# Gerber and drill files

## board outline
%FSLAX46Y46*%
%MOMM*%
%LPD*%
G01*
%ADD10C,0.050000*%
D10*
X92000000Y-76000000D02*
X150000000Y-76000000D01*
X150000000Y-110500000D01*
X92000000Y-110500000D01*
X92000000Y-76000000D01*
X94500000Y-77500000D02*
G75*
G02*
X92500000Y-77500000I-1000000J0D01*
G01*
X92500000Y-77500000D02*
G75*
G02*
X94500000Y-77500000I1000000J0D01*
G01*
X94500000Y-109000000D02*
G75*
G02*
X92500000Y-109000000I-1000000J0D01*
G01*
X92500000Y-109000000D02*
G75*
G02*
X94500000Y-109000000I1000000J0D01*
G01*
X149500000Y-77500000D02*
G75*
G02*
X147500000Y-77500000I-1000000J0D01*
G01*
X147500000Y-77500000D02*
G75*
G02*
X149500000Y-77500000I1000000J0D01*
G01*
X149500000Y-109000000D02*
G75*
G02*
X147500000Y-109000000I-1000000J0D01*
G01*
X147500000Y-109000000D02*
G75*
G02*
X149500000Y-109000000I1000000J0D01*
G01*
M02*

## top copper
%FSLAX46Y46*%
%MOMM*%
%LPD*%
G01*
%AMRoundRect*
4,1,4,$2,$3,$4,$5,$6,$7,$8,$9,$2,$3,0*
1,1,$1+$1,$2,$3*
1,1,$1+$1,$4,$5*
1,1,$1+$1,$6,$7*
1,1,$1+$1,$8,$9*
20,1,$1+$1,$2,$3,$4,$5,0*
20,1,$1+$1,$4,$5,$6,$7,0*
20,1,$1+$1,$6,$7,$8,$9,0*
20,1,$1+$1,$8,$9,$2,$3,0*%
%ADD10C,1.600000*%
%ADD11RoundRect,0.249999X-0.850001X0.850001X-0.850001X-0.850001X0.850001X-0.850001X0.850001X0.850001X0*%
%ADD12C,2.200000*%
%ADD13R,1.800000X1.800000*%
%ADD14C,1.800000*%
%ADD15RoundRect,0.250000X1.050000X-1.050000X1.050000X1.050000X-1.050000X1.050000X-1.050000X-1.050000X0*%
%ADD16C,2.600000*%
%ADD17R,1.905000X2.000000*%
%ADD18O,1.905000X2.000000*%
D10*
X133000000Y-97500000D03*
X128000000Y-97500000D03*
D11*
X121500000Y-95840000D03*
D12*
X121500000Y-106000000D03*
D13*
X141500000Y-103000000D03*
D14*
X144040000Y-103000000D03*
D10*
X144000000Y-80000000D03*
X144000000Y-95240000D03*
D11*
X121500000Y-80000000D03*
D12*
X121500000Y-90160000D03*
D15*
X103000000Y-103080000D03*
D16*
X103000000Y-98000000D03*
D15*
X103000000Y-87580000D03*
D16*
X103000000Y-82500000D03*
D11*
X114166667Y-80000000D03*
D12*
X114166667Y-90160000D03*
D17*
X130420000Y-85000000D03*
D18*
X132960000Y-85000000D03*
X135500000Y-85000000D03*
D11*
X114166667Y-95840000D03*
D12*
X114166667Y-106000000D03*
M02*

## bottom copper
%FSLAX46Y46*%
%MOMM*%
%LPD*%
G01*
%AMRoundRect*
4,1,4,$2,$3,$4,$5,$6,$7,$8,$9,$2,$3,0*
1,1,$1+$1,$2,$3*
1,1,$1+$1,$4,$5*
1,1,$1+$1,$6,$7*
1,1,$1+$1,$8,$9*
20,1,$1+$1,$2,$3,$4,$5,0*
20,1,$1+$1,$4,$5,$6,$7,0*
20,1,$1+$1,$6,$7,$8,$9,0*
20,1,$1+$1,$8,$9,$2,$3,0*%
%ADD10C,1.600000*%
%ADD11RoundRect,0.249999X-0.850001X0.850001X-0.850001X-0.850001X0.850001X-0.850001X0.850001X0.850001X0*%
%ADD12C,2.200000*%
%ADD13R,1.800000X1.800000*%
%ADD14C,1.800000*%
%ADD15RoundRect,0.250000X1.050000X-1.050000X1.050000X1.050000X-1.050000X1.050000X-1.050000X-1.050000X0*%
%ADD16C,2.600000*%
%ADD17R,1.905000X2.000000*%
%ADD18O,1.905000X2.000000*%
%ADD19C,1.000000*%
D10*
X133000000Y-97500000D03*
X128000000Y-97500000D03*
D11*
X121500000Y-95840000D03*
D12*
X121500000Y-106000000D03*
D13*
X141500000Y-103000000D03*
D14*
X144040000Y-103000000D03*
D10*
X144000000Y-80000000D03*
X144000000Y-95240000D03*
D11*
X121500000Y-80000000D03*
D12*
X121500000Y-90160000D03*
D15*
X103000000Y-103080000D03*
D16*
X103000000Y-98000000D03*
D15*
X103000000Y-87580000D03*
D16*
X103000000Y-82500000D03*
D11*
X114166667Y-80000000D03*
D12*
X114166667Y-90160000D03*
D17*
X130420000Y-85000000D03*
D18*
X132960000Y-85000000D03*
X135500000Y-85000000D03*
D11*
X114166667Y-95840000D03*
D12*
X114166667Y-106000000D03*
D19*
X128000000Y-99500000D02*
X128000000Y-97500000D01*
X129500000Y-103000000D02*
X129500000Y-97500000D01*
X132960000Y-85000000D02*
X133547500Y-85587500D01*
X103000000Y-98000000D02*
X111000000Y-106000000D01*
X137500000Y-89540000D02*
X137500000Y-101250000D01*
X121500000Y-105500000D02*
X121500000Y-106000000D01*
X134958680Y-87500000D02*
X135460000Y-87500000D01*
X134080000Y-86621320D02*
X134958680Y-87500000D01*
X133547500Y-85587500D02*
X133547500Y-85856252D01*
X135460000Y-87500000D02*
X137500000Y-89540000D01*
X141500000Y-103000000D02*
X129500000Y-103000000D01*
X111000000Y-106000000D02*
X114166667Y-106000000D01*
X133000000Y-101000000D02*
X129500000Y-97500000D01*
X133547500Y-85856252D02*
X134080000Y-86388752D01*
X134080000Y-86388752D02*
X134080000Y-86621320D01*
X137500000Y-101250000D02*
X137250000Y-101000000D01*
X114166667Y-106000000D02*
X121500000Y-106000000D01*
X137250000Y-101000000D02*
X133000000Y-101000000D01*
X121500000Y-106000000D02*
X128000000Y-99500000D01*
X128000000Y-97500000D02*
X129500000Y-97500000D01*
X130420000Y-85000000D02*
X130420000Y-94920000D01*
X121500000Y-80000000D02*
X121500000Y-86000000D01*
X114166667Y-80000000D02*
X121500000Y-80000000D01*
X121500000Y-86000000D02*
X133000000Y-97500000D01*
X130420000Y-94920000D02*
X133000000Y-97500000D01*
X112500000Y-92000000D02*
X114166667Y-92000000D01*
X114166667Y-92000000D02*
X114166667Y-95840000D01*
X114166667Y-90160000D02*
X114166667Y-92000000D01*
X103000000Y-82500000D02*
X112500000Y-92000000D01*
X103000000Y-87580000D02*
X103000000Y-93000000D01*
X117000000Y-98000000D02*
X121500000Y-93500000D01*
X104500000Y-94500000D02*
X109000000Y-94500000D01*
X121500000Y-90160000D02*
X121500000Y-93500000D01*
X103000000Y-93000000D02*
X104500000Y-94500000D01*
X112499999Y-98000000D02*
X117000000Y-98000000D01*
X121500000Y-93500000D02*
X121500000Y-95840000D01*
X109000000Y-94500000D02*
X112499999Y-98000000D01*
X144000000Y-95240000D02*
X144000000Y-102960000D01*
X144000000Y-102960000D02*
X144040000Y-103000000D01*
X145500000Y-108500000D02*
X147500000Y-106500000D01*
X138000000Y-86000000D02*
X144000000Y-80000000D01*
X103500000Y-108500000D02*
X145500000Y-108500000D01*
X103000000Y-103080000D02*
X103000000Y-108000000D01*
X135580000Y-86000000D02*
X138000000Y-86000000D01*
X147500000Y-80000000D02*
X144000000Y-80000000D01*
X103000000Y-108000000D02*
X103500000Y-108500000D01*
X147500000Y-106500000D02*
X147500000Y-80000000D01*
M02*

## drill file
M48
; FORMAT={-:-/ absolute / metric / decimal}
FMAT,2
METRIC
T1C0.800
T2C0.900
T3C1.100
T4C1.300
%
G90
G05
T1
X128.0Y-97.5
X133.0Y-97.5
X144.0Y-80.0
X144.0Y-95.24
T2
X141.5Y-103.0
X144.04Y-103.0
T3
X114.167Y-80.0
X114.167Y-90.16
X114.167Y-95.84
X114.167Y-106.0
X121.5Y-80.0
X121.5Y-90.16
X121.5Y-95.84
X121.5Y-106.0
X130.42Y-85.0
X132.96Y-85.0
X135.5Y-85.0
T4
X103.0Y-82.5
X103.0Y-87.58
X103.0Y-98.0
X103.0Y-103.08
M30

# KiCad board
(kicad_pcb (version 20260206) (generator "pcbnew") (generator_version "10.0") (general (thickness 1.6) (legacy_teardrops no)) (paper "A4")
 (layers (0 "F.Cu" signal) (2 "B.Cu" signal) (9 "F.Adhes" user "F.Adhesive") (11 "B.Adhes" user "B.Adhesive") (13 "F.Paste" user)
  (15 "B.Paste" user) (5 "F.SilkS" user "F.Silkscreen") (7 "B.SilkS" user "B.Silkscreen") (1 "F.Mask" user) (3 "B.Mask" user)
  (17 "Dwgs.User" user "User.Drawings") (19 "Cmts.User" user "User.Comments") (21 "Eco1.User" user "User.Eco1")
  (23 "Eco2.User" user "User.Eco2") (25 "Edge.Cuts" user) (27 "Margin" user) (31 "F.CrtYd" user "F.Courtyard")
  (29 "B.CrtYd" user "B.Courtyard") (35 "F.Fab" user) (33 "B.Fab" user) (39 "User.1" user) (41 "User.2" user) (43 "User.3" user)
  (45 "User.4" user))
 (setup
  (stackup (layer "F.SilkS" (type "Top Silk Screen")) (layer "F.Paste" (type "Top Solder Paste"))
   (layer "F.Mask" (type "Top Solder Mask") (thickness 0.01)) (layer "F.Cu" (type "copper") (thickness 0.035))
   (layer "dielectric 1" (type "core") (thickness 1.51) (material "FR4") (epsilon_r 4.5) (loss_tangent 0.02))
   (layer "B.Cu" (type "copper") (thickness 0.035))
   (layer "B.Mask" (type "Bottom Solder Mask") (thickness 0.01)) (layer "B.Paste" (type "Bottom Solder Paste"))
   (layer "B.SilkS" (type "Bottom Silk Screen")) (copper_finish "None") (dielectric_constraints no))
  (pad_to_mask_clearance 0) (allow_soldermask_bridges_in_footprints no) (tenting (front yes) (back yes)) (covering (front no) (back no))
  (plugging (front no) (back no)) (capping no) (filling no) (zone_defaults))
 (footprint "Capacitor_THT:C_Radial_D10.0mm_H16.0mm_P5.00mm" (layer "F.Cu") (at 133 97.5 180)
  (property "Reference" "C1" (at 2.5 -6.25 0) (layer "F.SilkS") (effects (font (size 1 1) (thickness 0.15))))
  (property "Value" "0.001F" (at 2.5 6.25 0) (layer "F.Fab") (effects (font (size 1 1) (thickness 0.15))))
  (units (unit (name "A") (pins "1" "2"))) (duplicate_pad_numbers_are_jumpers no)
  (pad "1" thru_hole circle (at 0 0 180) (size 1.6 1.6) (drill 0.8) (layers "*.Cu" "*.Mask") (remove_unused_layers no) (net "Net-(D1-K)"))
  (pad "2" thru_hole circle (at 5 0 180) (size 1.6 1.6) (drill 0.8) (layers "*.Cu" "*.Mask") (remove_unused_layers no) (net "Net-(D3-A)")))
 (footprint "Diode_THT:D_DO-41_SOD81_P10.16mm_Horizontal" (layer "F.Cu") (at 121.5 95.84 -90)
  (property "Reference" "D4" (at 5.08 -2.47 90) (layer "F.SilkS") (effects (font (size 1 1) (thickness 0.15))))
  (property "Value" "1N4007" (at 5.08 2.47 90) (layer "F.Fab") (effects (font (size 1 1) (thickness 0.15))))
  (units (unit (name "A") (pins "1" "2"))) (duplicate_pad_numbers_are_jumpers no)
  (pad "1" thru_hole roundrect (at 0 0 270) (size 2.2 2.2) (drill 1.1) (layers "*.Cu" "*.Mask") (remove_unused_layers no)
   (roundrect_rratio 0.113636) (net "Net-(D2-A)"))
  (pad "2" thru_hole circle (at 10.16 0 270) (size 2.2 2.2) (drill 1.1) (layers "*.Cu" "*.Mask") (remove_unused_layers no)
   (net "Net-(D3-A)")))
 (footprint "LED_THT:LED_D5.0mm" (layer "F.Cu") (at 141.5 103)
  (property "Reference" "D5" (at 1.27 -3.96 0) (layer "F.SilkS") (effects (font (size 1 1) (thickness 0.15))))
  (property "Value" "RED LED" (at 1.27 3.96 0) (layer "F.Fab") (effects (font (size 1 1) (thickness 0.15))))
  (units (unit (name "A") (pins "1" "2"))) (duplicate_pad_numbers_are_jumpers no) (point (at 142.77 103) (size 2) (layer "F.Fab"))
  (pad "1" thru_hole rect (at 0 0) (size 1.8 1.8) (drill 0.9) (layers "*.Cu" "*.Mask") (remove_unused_layers no) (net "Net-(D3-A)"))
  (pad "2" thru_hole circle (at 2.54 0) (size 1.8 1.8) (drill 0.9) (layers "*.Cu" "*.Mask") (remove_unused_layers no) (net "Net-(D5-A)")))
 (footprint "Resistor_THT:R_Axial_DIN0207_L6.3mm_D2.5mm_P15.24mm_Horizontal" (layer "F.Cu") (at 144 80 -90)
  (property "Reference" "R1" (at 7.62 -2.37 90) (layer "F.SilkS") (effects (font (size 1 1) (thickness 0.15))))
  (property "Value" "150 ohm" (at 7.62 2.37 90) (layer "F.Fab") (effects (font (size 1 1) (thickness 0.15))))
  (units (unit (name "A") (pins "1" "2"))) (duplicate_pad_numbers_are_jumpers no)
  (pad "1" thru_hole circle (at 0 0 270) (size 1.6 1.6) (drill 0.8) (layers "*.Cu" "*.Mask") (remove_unused_layers no)
   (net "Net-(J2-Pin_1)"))
  (pad "2" thru_hole circle (at 15.24 0 270) (size 1.6 1.6) (drill 0.8) (layers "*.Cu" "*.Mask") (remove_unused_layers no)
   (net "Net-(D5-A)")))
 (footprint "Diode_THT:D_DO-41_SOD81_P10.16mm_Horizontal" (layer "F.Cu") (at 121.5 80 -90)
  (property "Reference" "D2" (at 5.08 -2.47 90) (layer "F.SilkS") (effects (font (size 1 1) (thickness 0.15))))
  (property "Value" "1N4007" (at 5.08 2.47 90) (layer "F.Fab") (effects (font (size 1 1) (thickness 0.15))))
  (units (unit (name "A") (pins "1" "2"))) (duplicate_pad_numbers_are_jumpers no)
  (pad "1" thru_hole roundrect (at 0 0 270) (size 2.2 2.2) (drill 1.1) (layers "*.Cu" "*.Mask") (remove_unused_layers no)
   (roundrect_rratio 0.113636) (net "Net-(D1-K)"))
  (pad "2" thru_hole circle (at 10.16 0 270) (size 2.2 2.2) (drill 1.1) (layers "*.Cu" "*.Mask") (remove_unused_layers no)
   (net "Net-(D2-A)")))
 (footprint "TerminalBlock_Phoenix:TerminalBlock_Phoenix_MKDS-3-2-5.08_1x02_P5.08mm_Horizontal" (layer "F.Cu") (at 103 103.08 90)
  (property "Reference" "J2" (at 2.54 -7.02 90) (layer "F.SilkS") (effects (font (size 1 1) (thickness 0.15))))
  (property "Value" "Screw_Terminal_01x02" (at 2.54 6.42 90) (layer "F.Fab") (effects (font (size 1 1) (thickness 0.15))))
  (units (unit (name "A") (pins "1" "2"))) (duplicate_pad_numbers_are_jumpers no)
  (pad "1" thru_hole roundrect (at 0 0 90) (size 2.6 2.6) (drill 1.3) (layers "*.Cu" "*.Mask") (remove_unused_layers no)
   (roundrect_rratio 0.096154) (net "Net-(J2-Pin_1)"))
  (pad "2" thru_hole circle (at 5.08 0 90) (size 2.6 2.6) (drill 1.3) (layers "*.Cu" "*.Mask") (remove_unused_layers no) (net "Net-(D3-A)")))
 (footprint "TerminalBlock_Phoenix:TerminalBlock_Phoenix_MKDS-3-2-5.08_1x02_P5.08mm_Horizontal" (layer "F.Cu") (at 103 87.58 90)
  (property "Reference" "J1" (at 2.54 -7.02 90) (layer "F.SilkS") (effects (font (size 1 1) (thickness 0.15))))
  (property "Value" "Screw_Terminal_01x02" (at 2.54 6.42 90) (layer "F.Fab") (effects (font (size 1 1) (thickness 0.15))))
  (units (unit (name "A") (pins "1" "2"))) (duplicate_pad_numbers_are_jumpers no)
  (pad "1" thru_hole roundrect (at 0 0 90) (size 2.6 2.6) (drill 1.3) (layers "*.Cu" "*.Mask") (remove_unused_layers no)
   (roundrect_rratio 0.096154) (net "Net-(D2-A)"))
  (pad "2" thru_hole circle (at 5.08 0 90) (size 2.6 2.6) (drill 1.3) (layers "*.Cu" "*.Mask") (remove_unused_layers no) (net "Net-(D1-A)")))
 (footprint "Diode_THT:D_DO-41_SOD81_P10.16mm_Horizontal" (layer "F.Cu") (at 114.166667 80 -90)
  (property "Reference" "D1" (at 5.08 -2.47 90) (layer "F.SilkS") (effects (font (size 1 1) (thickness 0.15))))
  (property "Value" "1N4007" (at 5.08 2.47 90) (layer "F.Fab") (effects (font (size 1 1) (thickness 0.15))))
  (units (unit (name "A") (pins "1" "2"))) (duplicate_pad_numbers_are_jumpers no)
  (pad "1" thru_hole roundrect (at 0 0 270) (size 2.2 2.2) (drill 1.1) (layers "*.Cu" "*.Mask") (remove_unused_layers no)
   (roundrect_rratio 0.113636) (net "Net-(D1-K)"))
  (pad "2" thru_hole circle (at 10.16 0 270) (size 2.2 2.2) (drill 1.1) (layers "*.Cu" "*.Mask") (remove_unused_layers no)
   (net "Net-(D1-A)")))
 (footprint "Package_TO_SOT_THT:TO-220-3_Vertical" (layer "F.Cu") (at 130.42 85)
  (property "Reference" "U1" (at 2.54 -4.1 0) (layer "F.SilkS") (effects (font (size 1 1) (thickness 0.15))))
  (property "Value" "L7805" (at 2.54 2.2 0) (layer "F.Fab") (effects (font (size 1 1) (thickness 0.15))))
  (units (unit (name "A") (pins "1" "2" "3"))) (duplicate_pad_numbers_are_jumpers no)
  (pad "1" thru_hole rect (at 0 0) (size 1.905 2) (drill 1.1) (layers "*.Cu" "*.Mask") (remove_unused_layers no) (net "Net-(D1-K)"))
  (pad "2" thru_hole oval (at 2.54 0) (size 1.905 2) (drill 1.1) (layers "*.Cu" "*.Mask") (remove_unused_layers no) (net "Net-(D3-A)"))
  (pad "3" thru_hole oval (at 5.08 0) (size 1.905 2) (drill 1.1) (layers "*.Cu" "*.Mask") (remove_unused_layers no) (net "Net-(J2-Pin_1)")))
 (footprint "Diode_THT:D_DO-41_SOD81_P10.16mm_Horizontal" (layer "F.Cu") (at 114.166667 95.84 -90)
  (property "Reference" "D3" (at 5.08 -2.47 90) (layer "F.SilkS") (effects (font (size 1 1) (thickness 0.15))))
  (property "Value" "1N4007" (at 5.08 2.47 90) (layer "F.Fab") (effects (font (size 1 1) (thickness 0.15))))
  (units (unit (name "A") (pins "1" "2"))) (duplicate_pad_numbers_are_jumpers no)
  (pad "1" thru_hole roundrect (at 0 0 270) (size 2.2 2.2) (drill 1.1) (layers "*.Cu" "*.Mask") (remove_unused_layers no)
   (roundrect_rratio 0.113636) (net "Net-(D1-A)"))
  (pad "2" thru_hole circle (at 10.16 0 270) (size 2.2 2.2) (drill 1.1) (layers "*.Cu" "*.Mask") (remove_unused_layers no)
   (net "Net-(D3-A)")))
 (gr_rect (start 92 76) (end 150 110.5) (stroke (width 0.05) (type default)) (fill no) (layer "Edge.Cuts"))
 (gr_circle (center 93.5 77.5) (end 94.5 77.5) (stroke (width 0.05) (type default)) (fill no) (layer "Edge.Cuts"))
 (gr_circle (center 93.5 109) (end 94.5 109) (stroke (width 0.05) (type default)) (fill no) (layer "Edge.Cuts"))
 (gr_circle (center 148.5 77.5) (end 149.5 77.5) (stroke (width 0.05) (type default)) (fill no) (layer "Edge.Cuts"))
 (gr_circle (center 148.5 109) (end 149.5 109) (stroke (width 0.05) (type default)) (fill no) (layer "Edge.Cuts"))
 (segment (start 128 99.5) (end 128 97.5) (width 1) (layer "B.Cu") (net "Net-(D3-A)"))
 (segment (start 129.5 103) (end 129.5 97.5) (width 1) (layer "B.Cu") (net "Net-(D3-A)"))
 (segment (start 132.96 85) (end 133.5475 85.5875) (width 1) (layer "B.Cu") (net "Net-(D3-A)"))
 (segment (start 103 98) (end 111 106) (width 1) (layer "B.Cu") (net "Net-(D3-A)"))
 (segment (start 137.5 89.54) (end 137.5 101.25) (width 1) (layer "B.Cu") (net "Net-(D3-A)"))
 (segment (start 121.5 105.5) (end 121.5 106) (width 1) (layer "B.Cu") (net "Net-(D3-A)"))
 (segment (start 134.95868 87.5) (end 135.46 87.5) (width 1) (layer "B.Cu") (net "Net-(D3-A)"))
 (segment (start 134.08 86.62132) (end 134.95868 87.5) (width 1) (layer "B.Cu") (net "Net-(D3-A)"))
 (segment (start 133.5475 85.5875) (end 133.5475 85.856252) (width 1) (layer "B.Cu") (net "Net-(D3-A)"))
 (segment (start 135.46 87.5) (end 137.5 89.54) (width 1) (layer "B.Cu") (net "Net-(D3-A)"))
 (segment (start 141.5 103) (end 129.5 103) (width 1) (layer "B.Cu") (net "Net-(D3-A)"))
 (segment (start 111 106) (end 114.166667 106) (width 1) (layer "B.Cu") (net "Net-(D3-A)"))
 (segment (start 133 101) (end 129.5 97.5) (width 1) (layer "B.Cu") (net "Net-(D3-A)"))
 (segment (start 133.5475 85.856252) (end 134.08 86.388752) (width 1) (layer "B.Cu") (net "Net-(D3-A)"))
 (segment (start 134.08 86.388752) (end 134.08 86.62132) (width 1) (layer "B.Cu") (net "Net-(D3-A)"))
 (segment (start 137.5 101.25) (end 137.25 101) (width 1) (layer "B.Cu") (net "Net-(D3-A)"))
 (segment (start 114.166667 106) (end 121.5 106) (width 1) (layer "B.Cu") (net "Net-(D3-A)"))
 (segment (start 137.25 101) (end 133 101) (width 1) (layer "B.Cu") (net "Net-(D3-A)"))
 (segment (start 121.5 106) (end 128 99.5) (width 1) (layer "B.Cu") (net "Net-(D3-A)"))
 (segment (start 128 97.5) (end 129.5 97.5) (width 1) (layer "B.Cu") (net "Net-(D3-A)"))
 (segment (start 130.42 85) (end 130.42 94.92) (width 1) (layer "B.Cu") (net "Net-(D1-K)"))
 (segment (start 121.5 80) (end 121.5 86) (width 1) (layer "B.Cu") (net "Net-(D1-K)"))
 (segment (start 114.166667 80) (end 121.5 80) (width 1) (layer "B.Cu") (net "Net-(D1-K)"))
 (segment (start 121.5 86) (end 133 97.5) (width 1) (layer "B.Cu") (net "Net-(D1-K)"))
 (segment (start 130.42 94.92) (end 133 97.5) (width 1) (layer "B.Cu") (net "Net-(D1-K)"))
 (segment (start 112.5 92) (end 114.166667 92) (width 1) (layer "B.Cu") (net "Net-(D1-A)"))
 (segment (start 114.166667 92) (end 114.166667 95.84) (width 1) (layer "B.Cu") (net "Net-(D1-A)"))
 (segment (start 114.166667 90.16) (end 114.166667 92) (width 1) (layer "B.Cu") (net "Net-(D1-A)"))
 (segment (start 103 82.5) (end 112.5 92) (width 1) (layer "B.Cu") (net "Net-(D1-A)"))
 (segment (start 103 87.58) (end 103 93) (width 1) (layer "B.Cu") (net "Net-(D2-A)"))
 (segment (start 117 98) (end 121.5 93.5) (width 1) (layer "B.Cu") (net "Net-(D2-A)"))
 (segment (start 104.5 94.5) (end 109 94.5) (width 1) (layer "B.Cu") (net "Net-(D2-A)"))
 (segment (start 121.5 90.16) (end 121.5 93.5) (width 1) (layer "B.Cu") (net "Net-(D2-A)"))
 (segment (start 103 93) (end 104.5 94.5) (width 1) (layer "B.Cu") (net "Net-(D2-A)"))
 (segment (start 112.499999 98) (end 117 98) (width 1) (layer "B.Cu") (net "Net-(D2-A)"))
 (segment (start 121.5 93.5) (end 121.5 95.84) (width 1) (layer "B.Cu") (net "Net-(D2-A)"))
 (segment (start 109 94.5) (end 112.499999 98) (width 1) (layer "B.Cu") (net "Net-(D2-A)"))
 (segment (start 144 95.24) (end 144 102.96) (width 1) (layer "B.Cu") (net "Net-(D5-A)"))
 (segment (start 144 102.96) (end 144.04 103) (width 1) (layer "B.Cu") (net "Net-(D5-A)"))
 (segment (start 145.5 108.5) (end 147.5 106.5) (width 1) (layer "B.Cu") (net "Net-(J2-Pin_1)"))
 (segment (start 138 86) (end 144 80) (width 1) (layer "B.Cu") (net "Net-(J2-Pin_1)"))
 (segment (start 103.5 108.5) (end 145.5 108.5) (width 1) (layer "B.Cu") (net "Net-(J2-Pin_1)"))
 (segment (start 103 103.08) (end 103 108) (width 1) (layer "B.Cu") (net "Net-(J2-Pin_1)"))
 (segment (start 135.58 86) (end 138 86) (width 1) (layer "B.Cu") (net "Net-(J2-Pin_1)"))
 (segment (start 147.5 80) (end 144 80) (width 1) (layer "B.Cu") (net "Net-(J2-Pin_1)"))
 (segment (start 103 108) (end 103.5 108.5) (width 1) (layer "B.Cu") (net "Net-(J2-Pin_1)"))
 (segment (start 147.5 106.5) (end 147.5 80) (width 1) (layer "B.Cu") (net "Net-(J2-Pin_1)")))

